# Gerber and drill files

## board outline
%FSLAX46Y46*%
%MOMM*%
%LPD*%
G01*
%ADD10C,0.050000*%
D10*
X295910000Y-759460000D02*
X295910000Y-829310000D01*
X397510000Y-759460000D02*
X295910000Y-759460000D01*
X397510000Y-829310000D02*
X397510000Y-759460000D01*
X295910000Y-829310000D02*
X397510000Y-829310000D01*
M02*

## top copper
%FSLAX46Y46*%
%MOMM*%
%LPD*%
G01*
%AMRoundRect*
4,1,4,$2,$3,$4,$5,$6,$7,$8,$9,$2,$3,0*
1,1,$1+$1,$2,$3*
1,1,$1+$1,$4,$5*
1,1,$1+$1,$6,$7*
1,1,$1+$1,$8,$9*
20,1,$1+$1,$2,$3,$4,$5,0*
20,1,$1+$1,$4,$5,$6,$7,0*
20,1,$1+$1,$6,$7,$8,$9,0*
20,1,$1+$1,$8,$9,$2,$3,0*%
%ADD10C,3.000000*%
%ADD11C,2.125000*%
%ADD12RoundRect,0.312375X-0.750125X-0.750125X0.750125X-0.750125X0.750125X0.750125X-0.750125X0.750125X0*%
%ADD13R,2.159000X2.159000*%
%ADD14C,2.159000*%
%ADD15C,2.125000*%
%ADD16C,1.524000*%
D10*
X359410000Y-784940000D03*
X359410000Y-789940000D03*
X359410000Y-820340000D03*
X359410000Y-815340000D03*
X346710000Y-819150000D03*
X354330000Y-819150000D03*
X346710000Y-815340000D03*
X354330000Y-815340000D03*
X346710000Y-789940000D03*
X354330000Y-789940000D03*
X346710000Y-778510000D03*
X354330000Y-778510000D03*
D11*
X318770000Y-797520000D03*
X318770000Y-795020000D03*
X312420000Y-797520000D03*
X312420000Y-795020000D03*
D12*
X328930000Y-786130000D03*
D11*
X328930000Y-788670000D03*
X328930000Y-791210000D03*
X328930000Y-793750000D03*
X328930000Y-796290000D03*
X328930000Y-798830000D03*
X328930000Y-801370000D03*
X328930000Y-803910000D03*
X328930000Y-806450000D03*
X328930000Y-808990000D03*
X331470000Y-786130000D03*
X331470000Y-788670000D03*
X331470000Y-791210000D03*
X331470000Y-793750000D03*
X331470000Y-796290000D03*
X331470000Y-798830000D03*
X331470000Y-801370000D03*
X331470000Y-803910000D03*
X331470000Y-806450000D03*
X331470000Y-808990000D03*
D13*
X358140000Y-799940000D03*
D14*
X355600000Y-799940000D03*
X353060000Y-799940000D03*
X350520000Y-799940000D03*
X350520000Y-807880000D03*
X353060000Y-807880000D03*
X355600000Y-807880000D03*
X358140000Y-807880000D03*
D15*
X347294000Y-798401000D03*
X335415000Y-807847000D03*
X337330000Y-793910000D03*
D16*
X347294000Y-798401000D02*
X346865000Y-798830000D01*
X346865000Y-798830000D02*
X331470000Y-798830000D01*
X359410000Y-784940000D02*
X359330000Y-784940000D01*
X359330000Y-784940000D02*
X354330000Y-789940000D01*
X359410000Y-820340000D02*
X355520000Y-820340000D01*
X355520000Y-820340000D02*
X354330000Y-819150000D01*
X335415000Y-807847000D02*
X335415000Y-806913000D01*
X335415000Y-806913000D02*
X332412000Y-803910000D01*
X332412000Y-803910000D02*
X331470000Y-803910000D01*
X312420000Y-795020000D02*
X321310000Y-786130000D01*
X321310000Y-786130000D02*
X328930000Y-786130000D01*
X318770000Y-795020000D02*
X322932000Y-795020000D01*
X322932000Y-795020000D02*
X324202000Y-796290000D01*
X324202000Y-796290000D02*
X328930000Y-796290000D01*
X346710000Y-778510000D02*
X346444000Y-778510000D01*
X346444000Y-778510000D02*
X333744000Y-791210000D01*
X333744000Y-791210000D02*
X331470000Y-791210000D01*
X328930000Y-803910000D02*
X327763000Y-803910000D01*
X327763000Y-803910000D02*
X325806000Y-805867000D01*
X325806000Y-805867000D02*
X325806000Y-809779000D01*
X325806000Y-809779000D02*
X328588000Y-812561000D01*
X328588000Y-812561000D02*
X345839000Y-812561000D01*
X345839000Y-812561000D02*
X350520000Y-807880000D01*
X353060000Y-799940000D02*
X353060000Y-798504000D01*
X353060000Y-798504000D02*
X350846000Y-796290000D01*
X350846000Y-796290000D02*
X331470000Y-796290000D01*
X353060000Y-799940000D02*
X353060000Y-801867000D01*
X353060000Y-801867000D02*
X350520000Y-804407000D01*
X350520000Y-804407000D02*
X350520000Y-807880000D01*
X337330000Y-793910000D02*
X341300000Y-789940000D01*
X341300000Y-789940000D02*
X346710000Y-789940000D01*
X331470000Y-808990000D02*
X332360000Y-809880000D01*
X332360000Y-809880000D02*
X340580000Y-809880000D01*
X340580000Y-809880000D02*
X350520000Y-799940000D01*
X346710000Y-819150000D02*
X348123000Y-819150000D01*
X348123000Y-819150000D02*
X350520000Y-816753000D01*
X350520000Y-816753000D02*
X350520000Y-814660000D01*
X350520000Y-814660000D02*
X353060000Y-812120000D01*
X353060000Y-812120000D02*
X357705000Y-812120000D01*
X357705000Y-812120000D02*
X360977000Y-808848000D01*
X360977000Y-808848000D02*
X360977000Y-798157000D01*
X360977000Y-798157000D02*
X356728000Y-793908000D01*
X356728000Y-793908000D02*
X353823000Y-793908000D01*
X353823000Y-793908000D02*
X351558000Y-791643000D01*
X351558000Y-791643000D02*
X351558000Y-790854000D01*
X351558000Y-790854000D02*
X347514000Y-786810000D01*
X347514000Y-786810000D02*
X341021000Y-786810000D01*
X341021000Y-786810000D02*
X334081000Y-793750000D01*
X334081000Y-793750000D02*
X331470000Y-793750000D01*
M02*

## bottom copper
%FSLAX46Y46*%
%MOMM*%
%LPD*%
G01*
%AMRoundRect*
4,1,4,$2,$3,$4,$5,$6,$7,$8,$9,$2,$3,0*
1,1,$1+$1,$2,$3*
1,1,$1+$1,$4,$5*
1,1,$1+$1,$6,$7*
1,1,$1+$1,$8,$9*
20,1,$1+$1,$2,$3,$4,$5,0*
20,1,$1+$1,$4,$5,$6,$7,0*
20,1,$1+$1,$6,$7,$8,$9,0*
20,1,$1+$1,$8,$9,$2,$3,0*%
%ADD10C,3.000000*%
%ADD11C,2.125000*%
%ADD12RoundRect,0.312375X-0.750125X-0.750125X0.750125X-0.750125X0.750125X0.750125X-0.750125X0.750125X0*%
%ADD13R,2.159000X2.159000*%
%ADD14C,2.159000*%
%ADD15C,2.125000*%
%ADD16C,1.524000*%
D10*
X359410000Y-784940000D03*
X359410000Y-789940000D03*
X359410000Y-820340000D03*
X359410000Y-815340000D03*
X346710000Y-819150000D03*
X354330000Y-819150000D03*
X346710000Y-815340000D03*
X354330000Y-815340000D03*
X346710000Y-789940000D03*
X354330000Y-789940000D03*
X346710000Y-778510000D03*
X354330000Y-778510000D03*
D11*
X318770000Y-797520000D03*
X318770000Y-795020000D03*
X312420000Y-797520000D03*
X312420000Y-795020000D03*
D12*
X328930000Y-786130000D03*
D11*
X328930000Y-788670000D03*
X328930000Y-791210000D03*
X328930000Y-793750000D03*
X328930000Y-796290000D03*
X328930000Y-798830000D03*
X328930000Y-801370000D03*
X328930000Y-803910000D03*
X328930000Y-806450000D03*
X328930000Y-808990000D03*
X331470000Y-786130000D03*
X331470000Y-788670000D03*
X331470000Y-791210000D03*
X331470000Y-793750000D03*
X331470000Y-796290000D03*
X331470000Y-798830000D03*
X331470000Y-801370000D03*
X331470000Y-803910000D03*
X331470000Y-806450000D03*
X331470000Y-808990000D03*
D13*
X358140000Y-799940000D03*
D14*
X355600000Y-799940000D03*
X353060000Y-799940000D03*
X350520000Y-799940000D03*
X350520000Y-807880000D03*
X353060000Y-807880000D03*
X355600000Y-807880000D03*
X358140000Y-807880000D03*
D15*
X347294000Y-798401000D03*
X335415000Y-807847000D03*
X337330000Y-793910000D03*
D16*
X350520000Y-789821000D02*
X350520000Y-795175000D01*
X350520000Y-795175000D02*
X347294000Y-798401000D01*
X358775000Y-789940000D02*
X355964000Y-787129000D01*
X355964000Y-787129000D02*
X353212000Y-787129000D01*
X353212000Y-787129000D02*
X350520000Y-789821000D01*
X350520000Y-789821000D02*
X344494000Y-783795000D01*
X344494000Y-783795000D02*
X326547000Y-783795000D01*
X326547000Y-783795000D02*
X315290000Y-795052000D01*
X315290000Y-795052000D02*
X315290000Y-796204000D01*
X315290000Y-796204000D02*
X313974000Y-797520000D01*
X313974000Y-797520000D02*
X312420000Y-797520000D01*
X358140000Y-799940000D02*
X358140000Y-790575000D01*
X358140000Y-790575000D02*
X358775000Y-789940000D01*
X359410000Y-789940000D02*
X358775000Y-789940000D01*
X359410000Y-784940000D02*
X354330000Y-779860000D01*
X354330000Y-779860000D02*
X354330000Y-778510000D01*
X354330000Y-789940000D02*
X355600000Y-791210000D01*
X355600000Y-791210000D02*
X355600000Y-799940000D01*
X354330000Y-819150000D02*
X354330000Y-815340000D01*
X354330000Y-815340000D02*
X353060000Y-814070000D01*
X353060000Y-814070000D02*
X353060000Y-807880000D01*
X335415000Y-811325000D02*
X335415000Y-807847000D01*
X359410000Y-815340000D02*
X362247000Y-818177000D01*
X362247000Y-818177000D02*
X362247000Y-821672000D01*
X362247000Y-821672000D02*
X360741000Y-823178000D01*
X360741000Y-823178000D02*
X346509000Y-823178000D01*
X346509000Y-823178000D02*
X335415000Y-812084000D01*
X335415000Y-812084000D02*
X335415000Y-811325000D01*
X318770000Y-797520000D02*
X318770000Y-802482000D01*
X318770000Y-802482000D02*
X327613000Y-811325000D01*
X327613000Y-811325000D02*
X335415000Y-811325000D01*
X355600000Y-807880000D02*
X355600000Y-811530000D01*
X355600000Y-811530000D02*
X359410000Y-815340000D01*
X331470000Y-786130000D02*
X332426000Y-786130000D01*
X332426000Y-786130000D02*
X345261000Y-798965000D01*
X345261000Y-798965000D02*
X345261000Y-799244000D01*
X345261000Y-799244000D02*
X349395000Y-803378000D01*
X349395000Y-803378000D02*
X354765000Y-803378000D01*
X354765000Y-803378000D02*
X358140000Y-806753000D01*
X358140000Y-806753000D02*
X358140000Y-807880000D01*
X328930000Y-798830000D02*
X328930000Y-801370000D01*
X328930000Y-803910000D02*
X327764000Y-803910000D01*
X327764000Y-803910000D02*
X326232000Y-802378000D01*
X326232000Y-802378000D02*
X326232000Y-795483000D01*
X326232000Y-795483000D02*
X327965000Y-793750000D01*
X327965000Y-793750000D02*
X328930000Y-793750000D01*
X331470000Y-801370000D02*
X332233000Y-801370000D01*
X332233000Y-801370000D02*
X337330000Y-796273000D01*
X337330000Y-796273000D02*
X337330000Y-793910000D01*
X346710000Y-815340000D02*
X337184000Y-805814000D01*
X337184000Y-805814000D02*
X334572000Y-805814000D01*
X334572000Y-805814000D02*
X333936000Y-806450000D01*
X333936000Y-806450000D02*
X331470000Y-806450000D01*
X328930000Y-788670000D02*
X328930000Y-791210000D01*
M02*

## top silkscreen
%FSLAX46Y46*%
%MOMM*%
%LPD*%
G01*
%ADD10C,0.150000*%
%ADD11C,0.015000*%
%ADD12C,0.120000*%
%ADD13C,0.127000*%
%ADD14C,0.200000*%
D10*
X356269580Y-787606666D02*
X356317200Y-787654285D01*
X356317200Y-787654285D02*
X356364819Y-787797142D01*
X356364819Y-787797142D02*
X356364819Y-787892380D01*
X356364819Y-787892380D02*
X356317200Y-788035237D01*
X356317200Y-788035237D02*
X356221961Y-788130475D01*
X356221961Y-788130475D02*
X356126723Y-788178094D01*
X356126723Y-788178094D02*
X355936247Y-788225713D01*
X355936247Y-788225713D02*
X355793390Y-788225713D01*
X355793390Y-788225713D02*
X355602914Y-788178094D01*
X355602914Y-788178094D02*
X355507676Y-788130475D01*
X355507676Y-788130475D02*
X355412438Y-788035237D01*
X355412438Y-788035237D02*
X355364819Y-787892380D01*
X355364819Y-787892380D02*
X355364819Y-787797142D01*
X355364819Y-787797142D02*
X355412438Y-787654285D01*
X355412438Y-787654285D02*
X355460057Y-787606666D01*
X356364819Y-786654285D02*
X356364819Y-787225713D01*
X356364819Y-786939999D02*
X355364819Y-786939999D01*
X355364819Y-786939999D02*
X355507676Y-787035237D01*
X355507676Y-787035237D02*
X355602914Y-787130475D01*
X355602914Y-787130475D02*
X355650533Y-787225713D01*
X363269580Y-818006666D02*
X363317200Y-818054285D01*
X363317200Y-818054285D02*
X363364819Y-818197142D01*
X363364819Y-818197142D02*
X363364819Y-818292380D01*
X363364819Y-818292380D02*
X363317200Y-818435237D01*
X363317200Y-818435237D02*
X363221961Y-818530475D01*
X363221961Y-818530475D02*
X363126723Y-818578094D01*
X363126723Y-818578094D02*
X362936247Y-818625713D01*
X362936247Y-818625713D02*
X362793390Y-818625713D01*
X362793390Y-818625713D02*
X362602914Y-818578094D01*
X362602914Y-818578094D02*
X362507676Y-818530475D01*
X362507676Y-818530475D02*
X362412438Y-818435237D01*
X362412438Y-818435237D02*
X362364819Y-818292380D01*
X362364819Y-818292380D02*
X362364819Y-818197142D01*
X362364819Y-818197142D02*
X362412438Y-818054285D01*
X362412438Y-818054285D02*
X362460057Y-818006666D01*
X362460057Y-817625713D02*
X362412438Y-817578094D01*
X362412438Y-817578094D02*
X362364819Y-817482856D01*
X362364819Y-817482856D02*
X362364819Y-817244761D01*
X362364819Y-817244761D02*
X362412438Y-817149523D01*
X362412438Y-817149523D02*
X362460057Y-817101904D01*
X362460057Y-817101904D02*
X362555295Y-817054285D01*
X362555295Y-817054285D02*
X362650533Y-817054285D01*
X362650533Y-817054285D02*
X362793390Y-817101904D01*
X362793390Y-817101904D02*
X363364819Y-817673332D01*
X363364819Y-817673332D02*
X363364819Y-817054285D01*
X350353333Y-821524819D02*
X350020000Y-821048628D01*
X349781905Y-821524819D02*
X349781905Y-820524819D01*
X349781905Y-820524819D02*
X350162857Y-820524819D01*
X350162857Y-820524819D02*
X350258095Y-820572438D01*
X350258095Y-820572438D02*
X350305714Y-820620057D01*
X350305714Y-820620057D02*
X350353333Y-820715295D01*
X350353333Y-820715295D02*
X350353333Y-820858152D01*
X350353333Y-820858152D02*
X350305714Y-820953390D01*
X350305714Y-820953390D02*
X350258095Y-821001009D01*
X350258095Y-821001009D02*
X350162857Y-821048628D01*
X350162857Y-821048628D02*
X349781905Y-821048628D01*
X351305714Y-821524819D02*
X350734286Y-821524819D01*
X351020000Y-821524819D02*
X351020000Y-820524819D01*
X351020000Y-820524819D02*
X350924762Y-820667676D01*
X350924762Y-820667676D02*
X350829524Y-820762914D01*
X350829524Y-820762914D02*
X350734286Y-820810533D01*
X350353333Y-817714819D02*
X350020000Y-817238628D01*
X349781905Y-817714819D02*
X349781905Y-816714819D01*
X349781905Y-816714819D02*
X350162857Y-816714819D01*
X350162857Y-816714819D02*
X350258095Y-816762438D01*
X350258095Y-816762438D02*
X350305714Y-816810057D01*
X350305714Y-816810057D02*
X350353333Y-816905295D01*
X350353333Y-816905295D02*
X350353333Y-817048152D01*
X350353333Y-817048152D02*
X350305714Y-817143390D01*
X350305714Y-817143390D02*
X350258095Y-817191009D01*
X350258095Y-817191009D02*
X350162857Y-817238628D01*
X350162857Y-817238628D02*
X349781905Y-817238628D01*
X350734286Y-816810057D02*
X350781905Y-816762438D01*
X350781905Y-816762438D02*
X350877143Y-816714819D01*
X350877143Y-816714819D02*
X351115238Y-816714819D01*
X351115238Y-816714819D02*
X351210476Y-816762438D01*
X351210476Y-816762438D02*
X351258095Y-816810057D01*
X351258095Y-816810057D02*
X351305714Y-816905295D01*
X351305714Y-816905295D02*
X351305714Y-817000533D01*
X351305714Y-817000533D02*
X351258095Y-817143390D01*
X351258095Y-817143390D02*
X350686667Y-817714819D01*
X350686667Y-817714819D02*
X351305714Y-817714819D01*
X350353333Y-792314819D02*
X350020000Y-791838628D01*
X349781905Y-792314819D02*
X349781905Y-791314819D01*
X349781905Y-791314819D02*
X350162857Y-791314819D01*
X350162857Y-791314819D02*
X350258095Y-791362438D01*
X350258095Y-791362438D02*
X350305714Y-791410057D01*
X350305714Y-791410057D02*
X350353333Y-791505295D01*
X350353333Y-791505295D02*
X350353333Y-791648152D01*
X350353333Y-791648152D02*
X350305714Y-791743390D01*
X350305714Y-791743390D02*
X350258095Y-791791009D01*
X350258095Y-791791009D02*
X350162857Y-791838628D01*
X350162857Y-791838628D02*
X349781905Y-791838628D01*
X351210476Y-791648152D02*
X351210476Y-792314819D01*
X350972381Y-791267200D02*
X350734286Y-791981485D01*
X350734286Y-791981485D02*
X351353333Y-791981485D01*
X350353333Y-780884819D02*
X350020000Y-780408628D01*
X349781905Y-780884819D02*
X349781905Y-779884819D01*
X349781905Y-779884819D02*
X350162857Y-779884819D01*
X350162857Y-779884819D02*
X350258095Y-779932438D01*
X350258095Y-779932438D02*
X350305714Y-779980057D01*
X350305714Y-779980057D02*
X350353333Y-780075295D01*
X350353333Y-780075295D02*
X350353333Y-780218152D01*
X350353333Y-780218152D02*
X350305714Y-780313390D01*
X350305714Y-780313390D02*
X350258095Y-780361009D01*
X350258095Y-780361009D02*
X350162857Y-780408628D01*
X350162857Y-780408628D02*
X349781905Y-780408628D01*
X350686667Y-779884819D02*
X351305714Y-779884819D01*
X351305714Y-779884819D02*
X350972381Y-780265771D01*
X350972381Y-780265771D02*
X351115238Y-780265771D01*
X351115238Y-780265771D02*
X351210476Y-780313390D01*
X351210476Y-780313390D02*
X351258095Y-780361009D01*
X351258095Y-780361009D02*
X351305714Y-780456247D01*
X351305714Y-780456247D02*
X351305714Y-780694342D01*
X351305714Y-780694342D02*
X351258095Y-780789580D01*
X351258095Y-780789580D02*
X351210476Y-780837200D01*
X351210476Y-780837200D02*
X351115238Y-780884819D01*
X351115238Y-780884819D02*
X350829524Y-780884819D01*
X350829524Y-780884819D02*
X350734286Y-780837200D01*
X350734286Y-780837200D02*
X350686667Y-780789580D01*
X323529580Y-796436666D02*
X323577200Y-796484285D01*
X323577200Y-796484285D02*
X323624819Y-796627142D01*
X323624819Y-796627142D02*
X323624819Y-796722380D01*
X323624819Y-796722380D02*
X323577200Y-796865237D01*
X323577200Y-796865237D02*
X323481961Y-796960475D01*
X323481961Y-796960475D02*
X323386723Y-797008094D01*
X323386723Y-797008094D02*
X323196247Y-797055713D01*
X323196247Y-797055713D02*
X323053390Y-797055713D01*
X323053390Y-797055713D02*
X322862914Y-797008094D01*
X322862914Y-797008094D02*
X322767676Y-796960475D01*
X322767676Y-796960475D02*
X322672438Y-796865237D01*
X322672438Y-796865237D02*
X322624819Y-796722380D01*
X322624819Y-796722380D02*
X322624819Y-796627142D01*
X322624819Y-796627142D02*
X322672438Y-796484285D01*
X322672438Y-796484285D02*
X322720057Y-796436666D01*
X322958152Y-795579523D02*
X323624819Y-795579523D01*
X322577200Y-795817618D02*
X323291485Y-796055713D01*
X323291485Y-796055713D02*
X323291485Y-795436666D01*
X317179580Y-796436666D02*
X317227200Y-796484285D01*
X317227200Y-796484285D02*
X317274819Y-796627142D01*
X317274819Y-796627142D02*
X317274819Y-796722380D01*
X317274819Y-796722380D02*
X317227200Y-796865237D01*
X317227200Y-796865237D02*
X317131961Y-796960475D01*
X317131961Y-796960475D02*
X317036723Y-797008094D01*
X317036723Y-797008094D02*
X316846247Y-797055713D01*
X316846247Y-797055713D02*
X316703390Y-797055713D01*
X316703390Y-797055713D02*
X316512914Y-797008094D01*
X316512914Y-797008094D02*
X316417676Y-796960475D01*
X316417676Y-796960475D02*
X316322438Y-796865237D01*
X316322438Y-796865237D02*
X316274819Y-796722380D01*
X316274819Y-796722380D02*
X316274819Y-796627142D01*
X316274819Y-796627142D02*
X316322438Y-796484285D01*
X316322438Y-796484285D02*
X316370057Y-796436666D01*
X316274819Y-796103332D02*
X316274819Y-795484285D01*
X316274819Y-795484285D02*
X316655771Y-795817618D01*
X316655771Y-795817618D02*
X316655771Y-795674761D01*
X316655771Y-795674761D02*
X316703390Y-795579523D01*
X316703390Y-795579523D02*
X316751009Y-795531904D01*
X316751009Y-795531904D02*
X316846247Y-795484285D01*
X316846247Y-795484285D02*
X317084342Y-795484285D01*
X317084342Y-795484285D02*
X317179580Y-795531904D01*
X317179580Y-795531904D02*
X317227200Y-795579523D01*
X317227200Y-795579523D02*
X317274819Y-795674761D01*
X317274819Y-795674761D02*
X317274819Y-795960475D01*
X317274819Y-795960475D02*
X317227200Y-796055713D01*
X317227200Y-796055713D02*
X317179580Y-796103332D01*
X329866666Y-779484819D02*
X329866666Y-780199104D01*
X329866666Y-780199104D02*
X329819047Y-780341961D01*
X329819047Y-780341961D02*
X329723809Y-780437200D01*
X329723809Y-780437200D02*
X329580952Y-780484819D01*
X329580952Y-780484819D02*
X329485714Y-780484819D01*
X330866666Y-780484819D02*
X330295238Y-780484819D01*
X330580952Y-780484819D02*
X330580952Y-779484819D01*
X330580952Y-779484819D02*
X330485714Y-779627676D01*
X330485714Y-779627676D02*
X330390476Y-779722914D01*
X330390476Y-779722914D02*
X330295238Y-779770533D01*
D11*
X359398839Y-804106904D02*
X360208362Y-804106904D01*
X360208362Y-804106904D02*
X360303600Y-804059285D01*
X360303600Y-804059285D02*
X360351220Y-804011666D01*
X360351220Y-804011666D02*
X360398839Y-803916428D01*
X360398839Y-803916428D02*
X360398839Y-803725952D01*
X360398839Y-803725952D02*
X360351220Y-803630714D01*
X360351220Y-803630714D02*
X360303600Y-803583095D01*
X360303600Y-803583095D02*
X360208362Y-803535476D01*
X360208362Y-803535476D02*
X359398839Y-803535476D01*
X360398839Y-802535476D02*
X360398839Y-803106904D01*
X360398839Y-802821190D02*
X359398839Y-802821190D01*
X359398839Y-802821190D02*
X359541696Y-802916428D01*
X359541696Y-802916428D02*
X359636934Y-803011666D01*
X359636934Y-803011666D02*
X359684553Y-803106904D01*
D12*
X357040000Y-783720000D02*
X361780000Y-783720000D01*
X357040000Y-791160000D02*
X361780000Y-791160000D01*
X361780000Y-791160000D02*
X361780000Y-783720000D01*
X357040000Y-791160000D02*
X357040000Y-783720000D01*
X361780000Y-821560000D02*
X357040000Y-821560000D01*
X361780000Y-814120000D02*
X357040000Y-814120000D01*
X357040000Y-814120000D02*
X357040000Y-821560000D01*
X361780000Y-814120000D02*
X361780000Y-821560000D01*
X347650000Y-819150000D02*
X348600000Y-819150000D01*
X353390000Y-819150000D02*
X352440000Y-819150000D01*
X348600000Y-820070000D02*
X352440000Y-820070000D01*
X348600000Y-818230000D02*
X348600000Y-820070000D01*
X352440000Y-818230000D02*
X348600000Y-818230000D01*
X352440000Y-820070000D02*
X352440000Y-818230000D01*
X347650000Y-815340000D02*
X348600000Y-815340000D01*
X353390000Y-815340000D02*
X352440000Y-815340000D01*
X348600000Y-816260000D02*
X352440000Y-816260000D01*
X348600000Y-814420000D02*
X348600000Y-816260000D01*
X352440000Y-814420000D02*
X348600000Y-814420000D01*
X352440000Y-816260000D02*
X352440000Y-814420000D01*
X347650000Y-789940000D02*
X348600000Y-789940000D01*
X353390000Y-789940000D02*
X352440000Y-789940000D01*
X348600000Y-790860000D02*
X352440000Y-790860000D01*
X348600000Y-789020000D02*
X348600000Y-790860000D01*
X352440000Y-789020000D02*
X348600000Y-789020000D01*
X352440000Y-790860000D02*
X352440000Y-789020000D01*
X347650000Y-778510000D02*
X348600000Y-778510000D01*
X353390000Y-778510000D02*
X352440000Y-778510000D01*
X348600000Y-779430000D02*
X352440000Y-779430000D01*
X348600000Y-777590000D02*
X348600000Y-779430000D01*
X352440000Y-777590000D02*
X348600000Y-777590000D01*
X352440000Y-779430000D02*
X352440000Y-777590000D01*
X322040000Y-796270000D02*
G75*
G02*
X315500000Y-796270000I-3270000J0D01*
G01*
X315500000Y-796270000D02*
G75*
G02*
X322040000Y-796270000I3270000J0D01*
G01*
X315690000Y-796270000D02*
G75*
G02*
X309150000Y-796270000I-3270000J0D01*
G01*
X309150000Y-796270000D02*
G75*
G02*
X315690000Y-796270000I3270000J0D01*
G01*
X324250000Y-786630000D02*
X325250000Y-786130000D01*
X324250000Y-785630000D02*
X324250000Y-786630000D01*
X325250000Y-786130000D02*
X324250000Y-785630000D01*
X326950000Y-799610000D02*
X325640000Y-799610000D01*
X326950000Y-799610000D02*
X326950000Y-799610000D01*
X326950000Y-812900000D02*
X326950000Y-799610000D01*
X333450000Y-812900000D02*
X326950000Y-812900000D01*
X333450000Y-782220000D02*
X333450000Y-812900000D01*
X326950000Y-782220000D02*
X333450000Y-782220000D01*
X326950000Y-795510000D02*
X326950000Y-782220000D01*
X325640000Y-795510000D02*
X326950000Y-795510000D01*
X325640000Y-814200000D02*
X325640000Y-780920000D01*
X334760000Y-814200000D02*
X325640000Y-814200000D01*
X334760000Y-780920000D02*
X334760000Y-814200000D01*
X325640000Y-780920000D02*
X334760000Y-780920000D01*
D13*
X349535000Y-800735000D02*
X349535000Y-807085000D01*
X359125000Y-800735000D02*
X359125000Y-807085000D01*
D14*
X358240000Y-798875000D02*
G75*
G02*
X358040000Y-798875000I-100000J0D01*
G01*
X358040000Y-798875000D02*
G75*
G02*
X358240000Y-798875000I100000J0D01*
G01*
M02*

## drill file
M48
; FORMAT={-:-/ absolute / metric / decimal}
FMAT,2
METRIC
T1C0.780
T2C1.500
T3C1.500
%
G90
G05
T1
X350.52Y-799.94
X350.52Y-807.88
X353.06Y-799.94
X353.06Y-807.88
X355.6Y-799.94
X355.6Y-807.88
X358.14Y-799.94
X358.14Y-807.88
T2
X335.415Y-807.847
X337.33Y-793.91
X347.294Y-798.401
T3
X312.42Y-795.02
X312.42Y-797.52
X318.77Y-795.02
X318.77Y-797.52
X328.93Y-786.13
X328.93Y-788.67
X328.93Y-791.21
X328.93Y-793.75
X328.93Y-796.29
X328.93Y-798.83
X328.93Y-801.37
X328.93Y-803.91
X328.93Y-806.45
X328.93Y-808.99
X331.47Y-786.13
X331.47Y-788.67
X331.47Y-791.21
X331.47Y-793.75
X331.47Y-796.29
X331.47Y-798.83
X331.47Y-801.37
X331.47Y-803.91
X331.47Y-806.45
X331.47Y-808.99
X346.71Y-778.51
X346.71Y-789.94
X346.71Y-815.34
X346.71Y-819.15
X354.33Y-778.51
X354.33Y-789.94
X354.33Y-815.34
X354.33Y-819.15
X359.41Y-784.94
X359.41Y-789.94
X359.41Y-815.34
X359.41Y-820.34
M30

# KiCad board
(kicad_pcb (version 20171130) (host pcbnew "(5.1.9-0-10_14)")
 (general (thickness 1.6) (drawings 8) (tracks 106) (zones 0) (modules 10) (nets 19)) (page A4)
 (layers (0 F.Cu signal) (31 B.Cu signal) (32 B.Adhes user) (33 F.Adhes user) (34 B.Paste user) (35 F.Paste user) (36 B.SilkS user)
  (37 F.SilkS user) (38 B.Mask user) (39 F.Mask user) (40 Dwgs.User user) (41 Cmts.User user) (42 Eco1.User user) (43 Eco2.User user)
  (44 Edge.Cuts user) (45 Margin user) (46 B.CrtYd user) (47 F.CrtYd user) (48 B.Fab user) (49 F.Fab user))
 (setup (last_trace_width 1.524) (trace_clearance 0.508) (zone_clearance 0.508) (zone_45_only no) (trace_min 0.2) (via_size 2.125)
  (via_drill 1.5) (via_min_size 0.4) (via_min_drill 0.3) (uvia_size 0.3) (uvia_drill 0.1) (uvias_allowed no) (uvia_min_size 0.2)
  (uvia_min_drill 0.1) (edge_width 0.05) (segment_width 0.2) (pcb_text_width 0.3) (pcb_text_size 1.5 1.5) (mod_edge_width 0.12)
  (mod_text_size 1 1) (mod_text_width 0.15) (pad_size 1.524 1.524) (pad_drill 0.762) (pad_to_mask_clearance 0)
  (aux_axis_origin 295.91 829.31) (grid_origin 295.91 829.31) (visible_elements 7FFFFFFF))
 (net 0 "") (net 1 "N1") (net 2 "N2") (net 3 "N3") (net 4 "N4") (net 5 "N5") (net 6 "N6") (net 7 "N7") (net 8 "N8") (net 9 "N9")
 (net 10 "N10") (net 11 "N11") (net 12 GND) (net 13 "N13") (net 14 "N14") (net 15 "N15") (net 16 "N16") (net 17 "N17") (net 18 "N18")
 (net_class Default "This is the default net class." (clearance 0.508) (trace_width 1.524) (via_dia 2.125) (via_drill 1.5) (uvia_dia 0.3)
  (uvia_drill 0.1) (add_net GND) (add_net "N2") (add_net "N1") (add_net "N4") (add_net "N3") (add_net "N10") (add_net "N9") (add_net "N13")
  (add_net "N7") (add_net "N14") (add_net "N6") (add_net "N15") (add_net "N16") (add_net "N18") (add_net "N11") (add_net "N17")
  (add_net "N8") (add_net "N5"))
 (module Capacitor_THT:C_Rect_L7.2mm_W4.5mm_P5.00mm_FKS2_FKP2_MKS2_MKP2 (layer F.Cu) (at 359.41 789.94 90)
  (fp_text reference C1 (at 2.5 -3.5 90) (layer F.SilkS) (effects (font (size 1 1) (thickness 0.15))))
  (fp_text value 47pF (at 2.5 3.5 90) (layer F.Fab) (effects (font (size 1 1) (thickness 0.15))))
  (fp_line (start 6.22 -2.37) (end 6.22 2.37) (layer F.SilkS) (width 0.12))
  (fp_line (start -1.22 -2.37) (end -1.22 2.37) (layer F.SilkS) (width 0.12))
  (fp_line (start -1.22 2.37) (end 6.22 2.37) (layer F.SilkS) (width 0.12))
  (fp_line (start -1.22 -2.37) (end 6.22 -2.37) (layer F.SilkS) (width 0.12))
  (pad 2 thru_hole circle (at 5 0 90) (size 3 3) (drill 1.5) (layers *.Cu *.Mask) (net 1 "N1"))
  (pad 1 thru_hole circle (at 0 0 90) (size 3 3) (drill 1.5) (layers *.Cu *.Mask) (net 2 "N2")))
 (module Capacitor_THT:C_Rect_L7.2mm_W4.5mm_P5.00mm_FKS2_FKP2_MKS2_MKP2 (layer F.Cu) (at 359.41 815.34 270)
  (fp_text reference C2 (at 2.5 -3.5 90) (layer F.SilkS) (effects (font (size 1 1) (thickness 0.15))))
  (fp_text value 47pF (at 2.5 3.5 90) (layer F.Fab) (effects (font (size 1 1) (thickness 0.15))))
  (fp_line (start 6.22 -2.37) (end 6.22 2.37) (layer F.SilkS) (width 0.12))
  (fp_line (start -1.22 -2.37) (end -1.22 2.37) (layer F.SilkS) (width 0.12))
  (fp_line (start -1.22 2.37) (end 6.22 2.37) (layer F.SilkS) (width 0.12))
  (fp_line (start -1.22 -2.37) (end 6.22 -2.37) (layer F.SilkS) (width 0.12))
  (pad 2 thru_hole circle (at 5 0 270) (size 3 3) (drill 1.5) (layers *.Cu *.Mask) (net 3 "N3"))
  (pad 1 thru_hole circle (at 0 0 270) (size 3 3) (drill 1.5) (layers *.Cu *.Mask) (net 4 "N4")))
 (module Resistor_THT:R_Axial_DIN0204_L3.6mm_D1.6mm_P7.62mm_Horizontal (layer F.Cu) (at 354.33 819.15 180)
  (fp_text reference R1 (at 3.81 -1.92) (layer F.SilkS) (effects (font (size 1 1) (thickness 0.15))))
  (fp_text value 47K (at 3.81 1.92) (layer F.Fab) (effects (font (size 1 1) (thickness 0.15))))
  (fp_line (start 6.68 0) (end 5.73 0) (layer F.SilkS) (width 0.12))
  (fp_line (start 0.94 0) (end 1.89 0) (layer F.SilkS) (width 0.12))
  (fp_line (start 5.73 -0.92) (end 1.89 -0.92) (layer F.SilkS) (width 0.12))
  (fp_line (start 5.73 0.92) (end 5.73 -0.92) (layer F.SilkS) (width 0.12))
  (fp_line (start 1.89 0.92) (end 5.73 0.92) (layer F.SilkS) (width 0.12))
  (fp_line (start 1.89 -0.92) (end 1.89 0.92) (layer F.SilkS) (width 0.12))
  (pad 2 thru_hole circle (at 7.62 0 180) (size 3 3) (drill 1.5) (layers *.Cu *.Mask) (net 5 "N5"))
  (pad 1 thru_hole circle (at 0 0 180) (size 3 3) (drill 1.5) (layers *.Cu *.Mask) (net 3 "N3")))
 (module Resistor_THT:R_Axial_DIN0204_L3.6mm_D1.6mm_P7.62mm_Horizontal (layer F.Cu) (at 354.33 815.34 180)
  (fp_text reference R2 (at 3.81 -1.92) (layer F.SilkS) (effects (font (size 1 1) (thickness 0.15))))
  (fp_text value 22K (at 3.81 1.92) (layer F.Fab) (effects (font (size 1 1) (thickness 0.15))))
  (fp_line (start 6.68 0) (end 5.73 0) (layer F.SilkS) (width 0.12))
  (fp_line (start 0.94 0) (end 1.89 0) (layer F.SilkS) (width 0.12))
  (fp_line (start 5.73 -0.92) (end 1.89 -0.92) (layer F.SilkS) (width 0.12))
  (fp_line (start 5.73 0.92) (end 5.73 -0.92) (layer F.SilkS) (width 0.12))
  (fp_line (start 1.89 0.92) (end 5.73 0.92) (layer F.SilkS) (width 0.12))
  (fp_line (start 1.89 -0.92) (end 1.89 0.92) (layer F.SilkS) (width 0.12))
  (pad 2 thru_hole circle (at 7.62 0 180) (size 3 3) (drill 1.5) (layers *.Cu *.Mask) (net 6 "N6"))
  (pad 1 thru_hole circle (at 0 0 180) (size 3 3) (drill 1.5) (layers *.Cu *.Mask) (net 3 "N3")))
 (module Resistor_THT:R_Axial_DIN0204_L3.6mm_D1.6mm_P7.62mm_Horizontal (layer F.Cu) (at 354.33 789.94 180)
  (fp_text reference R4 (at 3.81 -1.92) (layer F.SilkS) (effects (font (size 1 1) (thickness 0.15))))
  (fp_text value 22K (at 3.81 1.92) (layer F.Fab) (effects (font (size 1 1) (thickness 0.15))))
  (fp_line (start 6.68 0) (end 5.73 0) (layer F.SilkS) (width 0.12))
  (fp_line (start 0.94 0) (end 1.89 0) (layer F.SilkS) (width 0.12))
  (fp_line (start 5.73 -0.92) (end 1.89 -0.92) (layer F.SilkS) (width 0.12))
  (fp_line (start 5.73 0.92) (end 5.73 -0.92) (layer F.SilkS) (width 0.12))
  (fp_line (start 1.89 0.92) (end 5.73 0.92) (layer F.SilkS) (width 0.12))
  (fp_line (start 1.89 -0.92) (end 1.89 0.92) (layer F.SilkS) (width 0.12))
  (pad 2 thru_hole circle (at 7.62 0 180) (size 3 3) (drill 1.5) (layers *.Cu *.Mask) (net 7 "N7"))
  (pad 1 thru_hole circle (at 0 0 180) (size 3 3) (drill 1.5) (layers *.Cu *.Mask) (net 1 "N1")))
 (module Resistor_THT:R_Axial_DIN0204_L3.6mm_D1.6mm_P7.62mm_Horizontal (layer F.Cu) (at 354.33 778.51 180)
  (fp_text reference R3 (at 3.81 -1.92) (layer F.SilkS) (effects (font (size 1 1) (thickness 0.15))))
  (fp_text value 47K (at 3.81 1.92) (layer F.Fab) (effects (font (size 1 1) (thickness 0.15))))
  (fp_line (start 6.68 0) (end 5.73 0) (layer F.SilkS) (width 0.12))
  (fp_line (start 0.94 0) (end 1.89 0) (layer F.SilkS) (width 0.12))
  (fp_line (start 5.73 -0.92) (end 1.89 -0.92) (layer F.SilkS) (width 0.12))
  (fp_line (start 5.73 0.92) (end 5.73 -0.92) (layer F.SilkS) (width 0.12))
  (fp_line (start 1.89 0.92) (end 5.73 0.92) (layer F.SilkS) (width 0.12))
  (fp_line (start 1.89 -0.92) (end 1.89 0.92) (layer F.SilkS) (width 0.12))
  (pad 2 thru_hole circle (at 7.62 0 180) (size 3 3) (drill 1.5) (layers *.Cu *.Mask) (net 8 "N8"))
  (pad 1 thru_hole circle (at 0 0 180) (size 3 3) (drill 1.5) (layers *.Cu *.Mask) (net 1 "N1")))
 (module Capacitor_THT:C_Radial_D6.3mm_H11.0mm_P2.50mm (layer F.Cu) (at 318.77 795.02 270)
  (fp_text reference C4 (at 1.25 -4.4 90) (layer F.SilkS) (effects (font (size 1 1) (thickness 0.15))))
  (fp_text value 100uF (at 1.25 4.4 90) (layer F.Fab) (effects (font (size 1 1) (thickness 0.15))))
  (fp_circle (center 1.25 0) (end 4.52 0) (layer F.SilkS) (width 0.12))
  (pad 2 thru_hole circle (at 2.5 0 270) (size 2.125 2.125) (drill 1.5) (layers *.Cu *.Mask) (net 4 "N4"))
  (pad 1 thru_hole circle (at 0 0 270) (size 2.125 2.125) (drill 1.5) (layers *.Cu *.Mask) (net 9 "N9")))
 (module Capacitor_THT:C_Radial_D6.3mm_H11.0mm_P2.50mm (layer F.Cu) (at 312.42 795.02 270)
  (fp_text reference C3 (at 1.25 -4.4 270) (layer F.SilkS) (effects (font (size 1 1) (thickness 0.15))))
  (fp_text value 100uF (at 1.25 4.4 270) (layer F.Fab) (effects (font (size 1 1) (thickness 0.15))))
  (fp_circle (center 1.25 0) (end 4.52 0) (layer F.SilkS) (width 0.12))
  (pad 2 thru_hole circle (at 2.5 0 270) (size 2.125 2.125) (drill 1.5) (layers *.Cu *.Mask) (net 2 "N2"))
  (pad 1 thru_hole circle (at 0 0 270) (size 2.125 2.125) (drill 1.5) (layers *.Cu *.Mask) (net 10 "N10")))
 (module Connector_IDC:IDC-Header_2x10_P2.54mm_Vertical (layer F.Cu) (at 328.93 786.13)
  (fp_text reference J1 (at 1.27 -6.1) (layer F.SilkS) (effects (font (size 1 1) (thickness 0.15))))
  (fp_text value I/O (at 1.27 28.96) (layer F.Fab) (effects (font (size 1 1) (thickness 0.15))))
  (fp_line (start -4.68 0.5) (end -3.68 0) (layer F.SilkS) (width 0.12))
  (fp_line (start -4.68 -0.5) (end -4.68 0.5) (layer F.SilkS) (width 0.12))
  (fp_line (start -3.68 0) (end -4.68 -0.5) (layer F.SilkS) (width 0.12))
  (fp_line (start -1.98 13.48) (end -3.29 13.48) (layer F.SilkS) (width 0.12))
  (fp_line (start -1.98 13.48) (end -1.98 13.48) (layer F.SilkS) (width 0.12))
  (fp_line (start -1.98 26.77) (end -1.98 13.48) (layer F.SilkS) (width 0.12))
  (fp_line (start 4.52 26.77) (end -1.98 26.77) (layer F.SilkS) (width 0.12))
  (fp_line (start 4.52 -3.91) (end 4.52 26.77) (layer F.SilkS) (width 0.12))
  (fp_line (start -1.98 -3.91) (end 4.52 -3.91) (layer F.SilkS) (width 0.12))
  (fp_line (start -1.98 9.38) (end -1.98 -3.91) (layer F.SilkS) (width 0.12))
  (fp_line (start -3.29 9.38) (end -1.98 9.38) (layer F.SilkS) (width 0.12))
  (fp_line (start -3.29 28.07) (end -3.29 -5.21) (layer F.SilkS) (width 0.12))
  (fp_line (start 5.83 28.07) (end -3.29 28.07) (layer F.SilkS) (width 0.12))
  (fp_line (start 5.83 -5.21) (end 5.83 28.07) (layer F.SilkS) (width 0.12))
  (fp_line (start -3.29 -5.21) (end 5.83 -5.21) (layer F.SilkS) (width 0.12))
  (pad 1 thru_hole roundrect (at 0 0) (size 2.125 2.125) (drill 1.5) (layers *.Cu *.Mask) (roundrect_rratio 0.147) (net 10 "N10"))
  (pad 3 thru_hole circle (at 0 2.54) (size 2.125 2.125) (drill 1.5) (layers *.Cu *.Mask) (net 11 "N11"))
  (pad 5 thru_hole circle (at 0 5.08) (size 2.125 2.125) (drill 1.5) (layers *.Cu *.Mask) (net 11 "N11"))
  (pad 7 thru_hole circle (at 0 7.62) (size 2.125 2.125) (drill 1.5) (layers *.Cu *.Mask) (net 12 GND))
  (pad 9 thru_hole circle (at 0 10.16) (size 2.125 2.125) (drill 1.5) (layers *.Cu *.Mask) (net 9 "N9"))
  (pad 11 thru_hole circle (at 0 12.7) (size 2.125 2.125) (drill 1.5) (layers *.Cu *.Mask) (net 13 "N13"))
  (pad 13 thru_hole circle (at 0 15.24) (size 2.125 2.125) (drill 1.5) (layers *.Cu *.Mask) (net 13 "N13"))
  (pad 15 thru_hole circle (at 0 17.78) (size 2.125 2.125) (drill 1.5) (layers *.Cu *.Mask) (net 12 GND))
  (pad 17 thru_hole circle (at 0 20.32) (size 2.125 2.125) (drill 1.5) (layers *.Cu *.Mask) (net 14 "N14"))
  (pad 19 thru_hole circle (at 0 22.86) (size 2.125 2.125) (drill 1.5) (layers *.Cu *.Mask) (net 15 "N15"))
  (pad 2 thru_hole circle (at 2.54 0) (size 2.125 2.125) (drill 1.5) (layers *.Cu *.Mask) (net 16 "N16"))
  (pad 4 thru_hole circle (at 2.54 2.54) (size 2.125 2.125) (drill 1.5) (layers *.Cu *.Mask) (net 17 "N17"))
  (pad 6 thru_hole circle (at 2.54 5.08) (size 2.125 2.125) (drill 1.5) (layers *.Cu *.Mask) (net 8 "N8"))
  (pad 8 thru_hole circle (at 2.54 7.62) (size 2.125 2.125) (drill 1.5) (layers *.Cu *.Mask) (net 5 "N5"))
  (pad 10 thru_hole circle (at 2.54 10.16) (size 2.125 2.125) (drill 1.5) (layers *.Cu *.Mask) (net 12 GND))
  (pad 12 thru_hole circle (at 2.54 12.7) (size 2.125 2.125) (drill 1.5) (layers *.Cu *.Mask) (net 2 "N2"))
  (pad 14 thru_hole circle (at 2.54 15.24) (size 2.125 2.125) (drill 1.5) (layers *.Cu *.Mask) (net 7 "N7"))
  (pad 16 thru_hole circle (at 2.54 17.78) (size 2.125 2.125) (drill 1.5) (layers *.Cu *.Mask) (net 4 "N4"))
  (pad 18 thru_hole circle (at 2.54 20.32) (size 2.125 2.125) (drill 1.5) (layers *.Cu *.Mask) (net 6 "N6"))
  (pad 20 thru_hole circle (at 2.54 22.86) (size 2.125 2.125) (drill 1.5) (layers *.Cu *.Mask) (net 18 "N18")))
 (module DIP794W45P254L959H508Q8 (layer F.Cu) (at 354.33 803.91 270)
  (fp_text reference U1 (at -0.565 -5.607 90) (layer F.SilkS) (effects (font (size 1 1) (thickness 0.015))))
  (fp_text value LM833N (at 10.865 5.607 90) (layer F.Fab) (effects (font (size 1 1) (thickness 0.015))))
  (fp_line (start -3.175 4.795) (end 3.175 4.795) (layer F.SilkS) (width 0.127))
  (fp_line (start -3.175 -4.795) (end 3.175 -4.795) (layer F.SilkS) (width 0.127))
  (fp_circle (center -5.035 -3.81) (end -4.935 -3.81) (layer F.SilkS) (width 0.2))
  (pad 1 thru_hole rect (at -3.97 -3.81 270) (size 2.159 2.159) (drill 0.78) (layers *.Cu *.Mask) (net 2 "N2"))
  (pad 2 thru_hole circle (at -3.97 -1.27 270) (size 2.159 2.159) (drill 0.78) (layers *.Cu *.Mask) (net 1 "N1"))
  (pad 3 thru_hole circle (at -3.97 1.27 270) (size 2.159 2.159) (drill 0.78) (layers *.Cu *.Mask) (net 12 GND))
  (pad 4 thru_hole circle (at -3.97 3.81 270) (size 2.159 2.159) (drill 0.78) (layers *.Cu *.Mask) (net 18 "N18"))
  (pad 5 thru_hole circle (at 3.97 3.81 270) (size 2.159 2.159) (drill 0.78) (layers *.Cu *.Mask) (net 12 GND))
  (pad 6 thru_hole circle (at 3.97 1.27 270) (size 2.159 2.159) (drill 0.78) (layers *.Cu *.Mask) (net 3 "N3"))
  (pad 7 thru_hole circle (at 3.97 -1.27 270) (size 2.159 2.159) (drill 0.78) (layers *.Cu *.Mask) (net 4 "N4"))
  (pad 8 thru_hole circle (at 3.97 -3.81 270) (size 2.159 2.159) (drill 0.78) (layers *.Cu *.Mask) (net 16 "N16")))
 (gr_line (start 295.91 759.46) (end 295.91 829.31) (layer Edge.Cuts) (width 0.05))
 (gr_line (start 397.51 759.46) (end 295.91 759.46) (layer Edge.Cuts) (width 0.05))
 (gr_line (start 397.51 829.31) (end 397.51 759.46) (layer Edge.Cuts) (width 0.05))
 (gr_line (start 295.91 829.31) (end 397.51 829.31) (layer Edge.Cuts) (width 0.05))
 (segment (start 350.52 789.821) (end 350.52 795.175) (width 1.524) (layer B.Cu) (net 2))
 (segment (start 350.52 795.175) (end 347.294 798.401) (width 1.524) (layer B.Cu) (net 2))
 (segment (start 358.775 789.94) (end 355.964 787.129) (width 1.524) (layer B.Cu) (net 2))
 (segment (start 355.964 787.129) (end 353.212 787.129) (width 1.524) (layer B.Cu) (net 2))
 (segment (start 353.212 787.129) (end 350.52 789.821) (width 1.524) (layer B.Cu) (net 2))
 (segment (start 350.52 789.821) (end 344.494 783.795) (width 1.524) (layer B.Cu) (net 2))
 (segment (start 344.494 783.795) (end 326.547 783.795) (width 1.524) (layer B.Cu) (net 2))
 (segment (start 326.547 783.795) (end 315.29 795.052) (width 1.524) (layer B.Cu) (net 2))
 (segment (start 315.29 795.052) (end 315.29 796.204) (width 1.524) (layer B.Cu) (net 2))
 (segment (start 315.29 796.204) (end 313.974 797.52) (width 1.524) (layer B.Cu) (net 2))
 (segment (start 313.974 797.52) (end 312.42 797.52) (width 1.524) (layer B.Cu) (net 2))
 (segment (start 358.14 799.94) (end 358.14 790.575) (width 1.524) (layer B.Cu) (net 2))
 (segment (start 358.14 790.575) (end 358.775 789.94) (width 1.524) (layer B.Cu) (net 2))
 (segment (start 359.41 789.94) (end 358.775 789.94) (width 1.524) (layer B.Cu) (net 2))
 (segment (start 347.294 798.401) (end 346.865 798.83) (width 1.524) (layer F.Cu) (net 2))
 (segment (start 346.865 798.83) (end 331.47 798.83) (width 1.524) (layer F.Cu) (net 2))
 (via (at 347.294 798.401) (size 2.125) (drill 1.5) (layers F.Cu B.Cu) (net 2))
 (segment (start 359.41 784.94) (end 359.33 784.94) (width 1.524) (layer F.Cu) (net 1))
 (segment (start 359.33 784.94) (end 354.33 789.94) (width 1.524) (layer F.Cu) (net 1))
 (segment (start 359.41 784.94) (end 354.33 779.86) (width 1.524) (layer B.Cu) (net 1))
 (segment (start 354.33 779.86) (end 354.33 778.51) (width 1.524) (layer B.Cu) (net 1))
 (segment (start 354.33 789.94) (end 355.6 791.21) (width 1.524) (layer B.Cu) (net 1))
 (segment (start 355.6 791.21) (end 355.6 799.94) (width 1.524) (layer B.Cu) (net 1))
 (segment (start 359.41 820.34) (end 355.52 820.34) (width 1.524) (layer F.Cu) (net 3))
 (segment (start 355.52 820.34) (end 354.33 819.15) (width 1.524) (layer F.Cu) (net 3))
 (segment (start 354.33 819.15) (end 354.33 815.34) (width 1.524) (layer B.Cu) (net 3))
 (segment (start 354.33 815.34) (end 353.06 814.07) (width 1.524) (layer B.Cu) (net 3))
 (segment (start 353.06 814.07) (end 353.06 807.88) (width 1.524) (layer B.Cu) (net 3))
 (segment (start 335.415 811.325) (end 335.415 807.847) (width 1.524) (layer B.Cu) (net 4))
 (segment (start 359.41 815.34) (end 362.247 818.177) (width 1.524) (layer B.Cu) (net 4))
 (segment (start 362.247 818.177) (end 362.247 821.672) (width 1.524) (layer B.Cu) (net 4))
 (segment (start 362.247 821.672) (end 360.741 823.178) (width 1.524) (layer B.Cu) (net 4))
 (segment (start 360.741 823.178) (end 346.509 823.178) (width 1.524) (layer B.Cu) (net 4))
 (segment (start 346.509 823.178) (end 335.415 812.084) (width 1.524) (layer B.Cu) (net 4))
 (segment (start 335.415 812.084) (end 335.415 811.325) (width 1.524) (layer B.Cu) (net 4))
 (segment (start 318.77 797.52) (end 318.77 802.482) (width 1.524) (layer B.Cu) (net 4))
 (segment (start 318.77 802.482) (end 327.613 811.325) (width 1.524) (layer B.Cu) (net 4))
 (segment (start 327.613 811.325) (end 335.415 811.325) (width 1.524) (layer B.Cu) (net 4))
 (segment (start 355.6 807.88) (end 355.6 811.53) (width 1.524) (layer B.Cu) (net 4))
 (segment (start 355.6 811.53) (end 359.41 815.34) (width 1.524) (layer B.Cu) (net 4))
 (segment (start 335.415 807.847) (end 335.415 806.913) (width 1.524) (layer F.Cu) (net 4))
 (segment (start 335.415 806.913) (end 332.412 803.91) (width 1.524) (layer F.Cu) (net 4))
 (segment (start 332.412 803.91) (end 331.47 803.91) (width 1.524) (layer F.Cu) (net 4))
 (via (at 335.415 807.847) (size 2.125) (drill 1.5) (layers F.Cu B.Cu) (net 4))
 (segment (start 312.42 795.02) (end 321.31 786.13) (width 1.524) (layer F.Cu) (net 10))
 (segment (start 321.31 786.13) (end 328.93 786.13) (width 1.524) (layer F.Cu) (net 10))
 (segment (start 318.77 795.02) (end 322.932 795.02) (width 1.524) (layer F.Cu) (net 9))
 (segment (start 322.932 795.02) (end 324.202 796.29) (width 1.524) (layer F.Cu) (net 9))
 (segment (start 324.202 796.29) (end 328.93 796.29) (width 1.524) (layer F.Cu) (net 9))
 (segment (start 331.47 786.13) (end 332.426 786.13) (width 1.524) (layer B.Cu) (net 16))
 (segment (start 332.426 786.13) (end 345.261 798.965) (width 1.524) (layer B.Cu) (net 16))
 (segment (start 345.261 798.965) (end 345.261 799.244) (width 1.524) (layer B.Cu) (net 16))
 (segment (start 345.261 799.244) (end 349.395 803.378) (width 1.524) (layer B.Cu) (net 16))
 (segment (start 349.395 803.378) (end 354.765 803.378) (width 1.524) (layer B.Cu) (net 16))
 (segment (start 354.765 803.378) (end 358.14 806.753) (width 1.524) (layer B.Cu) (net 16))
 (segment (start 358.14 806.753) (end 358.14 807.88) (width 1.524) (layer B.Cu) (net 16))
 (segment (start 346.71 778.51) (end 346.444 778.51) (width 1.524) (layer F.Cu) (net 8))
 (segment (start 346.444 778.51) (end 333.744 791.21) (width 1.524) (layer F.Cu) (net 8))
 (segment (start 333.744 791.21) (end 331.47 791.21) (width 1.524) (layer F.Cu) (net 8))
 (segment (start 328.93 798.83) (end 328.93 801.37) (width 1.524) (layer B.Cu) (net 13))
 (segment (start 328.93 803.91) (end 327.764 803.91) (width 1.524) (layer B.Cu) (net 12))
 (segment (start 327.764 803.91) (end 326.232 802.378) (width 1.524) (layer B.Cu) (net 12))
 (segment (start 326.232 802.378) (end 326.232 795.483) (width 1.524) (layer B.Cu) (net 12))
 (segment (start 326.232 795.483) (end 327.965 793.75) (width 1.524) (layer B.Cu) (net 12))
 (segment (start 327.965 793.75) (end 328.93 793.75) (width 1.524) (layer B.Cu) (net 12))
 (segment (start 328.93 803.91) (end 327.763 803.91) (width 1.524) (layer F.Cu) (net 12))
 (segment (start 327.763 803.91) (end 325.806 805.867) (width 1.524) (layer F.Cu) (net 12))
 (segment (start 325.806 805.867) (end 325.806 809.779) (width 1.524) (layer F.Cu) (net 12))
 (segment (start 325.806 809.779) (end 328.588 812.561) (width 1.524) (layer F.Cu) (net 12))
 (segment (start 328.588 812.561) (end 345.839 812.561) (width 1.524) (layer F.Cu) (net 12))
 (segment (start 345.839 812.561) (end 350.52 807.88) (width 1.524) (layer F.Cu) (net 12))
 (segment (start 353.06 799.94) (end 353.06 798.504) (width 1.524) (layer F.Cu) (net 12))
 (segment (start 353.06 798.504) (end 350.846 796.29) (width 1.524) (layer F.Cu) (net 12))
 (segment (start 350.846 796.29) (end 331.47 796.29) (width 1.524) (layer F.Cu) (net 12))
 (segment (start 353.06 799.94) (end 353.06 801.867) (width 1.524) (layer F.Cu) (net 12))
 (segment (start 353.06 801.867) (end 350.52 804.407) (width 1.524) (layer F.Cu) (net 12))
 (segment (start 350.52 804.407) (end 350.52 807.88) (width 1.524) (layer F.Cu) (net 12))
 (segment (start 337.33 793.91) (end 341.3 789.94) (width 1.524) (layer F.Cu) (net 7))
 (segment (start 341.3 789.94) (end 346.71 789.94) (width 1.524) (layer F.Cu) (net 7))
 (segment (start 331.47 801.37) (end 332.233 801.37) (width 1.524) (layer B.Cu) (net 7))
 (segment (start 332.233 801.37) (end 337.33 796.273) (width 1.524) (layer B.Cu) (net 7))
 (segment (start 337.33 796.273) (end 337.33 793.91) (width 1.524) (layer B.Cu) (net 7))
 (via (at 337.33 793.91) (size 2.125) (drill 1.5) (layers F.Cu B.Cu) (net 7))
 (segment (start 346.71 815.34) (end 337.184 805.814) (width 1.524) (layer B.Cu) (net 6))
 (segment (start 337.184 805.814) (end 334.572 805.814) (width 1.524) (layer B.Cu) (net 6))
 (segment (start 334.572 805.814) (end 333.936 806.45) (width 1.524) (layer B.Cu) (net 6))
 (segment (start 333.936 806.45) (end 331.47 806.45) (width 1.524) (layer B.Cu) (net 6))
 (segment (start 331.47 808.99) (end 332.36 809.88) (width 1.524) (layer F.Cu) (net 18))
 (segment (start 332.36 809.88) (end 340.58 809.88) (width 1.524) (layer F.Cu) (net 18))
 (segment (start 340.58 809.88) (end 350.52 799.94) (width 1.524) (layer F.Cu) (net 18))
 (segment (start 328.93 788.67) (end 328.93 791.21) (width 1.524) (layer B.Cu) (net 11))
 (segment (start 346.71 819.15) (end 348.123 819.15) (width 1.524) (layer F.Cu) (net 5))
 (segment (start 348.123 819.15) (end 350.52 816.753) (width 1.524) (layer F.Cu) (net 5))
 (segment (start 350.52 816.753) (end 350.52 814.66) (width 1.524) (layer F.Cu) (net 5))
 (segment (start 350.52 814.66) (end 353.06 812.12) (width 1.524) (layer F.Cu) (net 5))
 (segment (start 353.06 812.12) (end 357.705 812.12) (width 1.524) (layer F.Cu) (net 5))
 (segment (start 357.705 812.12) (end 360.977 808.848) (width 1.524) (layer F.Cu) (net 5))
 (segment (start 360.977 808.848) (end 360.977 798.157) (width 1.524) (layer F.Cu) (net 5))
 (segment (start 360.977 798.157) (end 356.728 793.908) (width 1.524) (layer F.Cu) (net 5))
 (segment (start 356.728 793.908) (end 353.823 793.908) (width 1.524) (layer F.Cu) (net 5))
 (segment (start 353.823 793.908) (end 351.558 791.643) (width 1.524) (layer F.Cu) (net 5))
 (segment (start 351.558 791.643) (end 351.558 790.854) (width 1.524) (layer F.Cu) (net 5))
 (segment (start 351.558 790.854) (end 347.514 786.81) (width 1.524) (layer F.Cu) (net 5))
 (segment (start 347.514 786.81) (end 341.021 786.81) (width 1.524) (layer F.Cu) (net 5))
 (segment (start 341.021 786.81) (end 334.081 793.75) (width 1.524) (layer F.Cu) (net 5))
 (segment (start 334.081 793.75) (end 331.47 793.75) (width 1.524) (layer F.Cu) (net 5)))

